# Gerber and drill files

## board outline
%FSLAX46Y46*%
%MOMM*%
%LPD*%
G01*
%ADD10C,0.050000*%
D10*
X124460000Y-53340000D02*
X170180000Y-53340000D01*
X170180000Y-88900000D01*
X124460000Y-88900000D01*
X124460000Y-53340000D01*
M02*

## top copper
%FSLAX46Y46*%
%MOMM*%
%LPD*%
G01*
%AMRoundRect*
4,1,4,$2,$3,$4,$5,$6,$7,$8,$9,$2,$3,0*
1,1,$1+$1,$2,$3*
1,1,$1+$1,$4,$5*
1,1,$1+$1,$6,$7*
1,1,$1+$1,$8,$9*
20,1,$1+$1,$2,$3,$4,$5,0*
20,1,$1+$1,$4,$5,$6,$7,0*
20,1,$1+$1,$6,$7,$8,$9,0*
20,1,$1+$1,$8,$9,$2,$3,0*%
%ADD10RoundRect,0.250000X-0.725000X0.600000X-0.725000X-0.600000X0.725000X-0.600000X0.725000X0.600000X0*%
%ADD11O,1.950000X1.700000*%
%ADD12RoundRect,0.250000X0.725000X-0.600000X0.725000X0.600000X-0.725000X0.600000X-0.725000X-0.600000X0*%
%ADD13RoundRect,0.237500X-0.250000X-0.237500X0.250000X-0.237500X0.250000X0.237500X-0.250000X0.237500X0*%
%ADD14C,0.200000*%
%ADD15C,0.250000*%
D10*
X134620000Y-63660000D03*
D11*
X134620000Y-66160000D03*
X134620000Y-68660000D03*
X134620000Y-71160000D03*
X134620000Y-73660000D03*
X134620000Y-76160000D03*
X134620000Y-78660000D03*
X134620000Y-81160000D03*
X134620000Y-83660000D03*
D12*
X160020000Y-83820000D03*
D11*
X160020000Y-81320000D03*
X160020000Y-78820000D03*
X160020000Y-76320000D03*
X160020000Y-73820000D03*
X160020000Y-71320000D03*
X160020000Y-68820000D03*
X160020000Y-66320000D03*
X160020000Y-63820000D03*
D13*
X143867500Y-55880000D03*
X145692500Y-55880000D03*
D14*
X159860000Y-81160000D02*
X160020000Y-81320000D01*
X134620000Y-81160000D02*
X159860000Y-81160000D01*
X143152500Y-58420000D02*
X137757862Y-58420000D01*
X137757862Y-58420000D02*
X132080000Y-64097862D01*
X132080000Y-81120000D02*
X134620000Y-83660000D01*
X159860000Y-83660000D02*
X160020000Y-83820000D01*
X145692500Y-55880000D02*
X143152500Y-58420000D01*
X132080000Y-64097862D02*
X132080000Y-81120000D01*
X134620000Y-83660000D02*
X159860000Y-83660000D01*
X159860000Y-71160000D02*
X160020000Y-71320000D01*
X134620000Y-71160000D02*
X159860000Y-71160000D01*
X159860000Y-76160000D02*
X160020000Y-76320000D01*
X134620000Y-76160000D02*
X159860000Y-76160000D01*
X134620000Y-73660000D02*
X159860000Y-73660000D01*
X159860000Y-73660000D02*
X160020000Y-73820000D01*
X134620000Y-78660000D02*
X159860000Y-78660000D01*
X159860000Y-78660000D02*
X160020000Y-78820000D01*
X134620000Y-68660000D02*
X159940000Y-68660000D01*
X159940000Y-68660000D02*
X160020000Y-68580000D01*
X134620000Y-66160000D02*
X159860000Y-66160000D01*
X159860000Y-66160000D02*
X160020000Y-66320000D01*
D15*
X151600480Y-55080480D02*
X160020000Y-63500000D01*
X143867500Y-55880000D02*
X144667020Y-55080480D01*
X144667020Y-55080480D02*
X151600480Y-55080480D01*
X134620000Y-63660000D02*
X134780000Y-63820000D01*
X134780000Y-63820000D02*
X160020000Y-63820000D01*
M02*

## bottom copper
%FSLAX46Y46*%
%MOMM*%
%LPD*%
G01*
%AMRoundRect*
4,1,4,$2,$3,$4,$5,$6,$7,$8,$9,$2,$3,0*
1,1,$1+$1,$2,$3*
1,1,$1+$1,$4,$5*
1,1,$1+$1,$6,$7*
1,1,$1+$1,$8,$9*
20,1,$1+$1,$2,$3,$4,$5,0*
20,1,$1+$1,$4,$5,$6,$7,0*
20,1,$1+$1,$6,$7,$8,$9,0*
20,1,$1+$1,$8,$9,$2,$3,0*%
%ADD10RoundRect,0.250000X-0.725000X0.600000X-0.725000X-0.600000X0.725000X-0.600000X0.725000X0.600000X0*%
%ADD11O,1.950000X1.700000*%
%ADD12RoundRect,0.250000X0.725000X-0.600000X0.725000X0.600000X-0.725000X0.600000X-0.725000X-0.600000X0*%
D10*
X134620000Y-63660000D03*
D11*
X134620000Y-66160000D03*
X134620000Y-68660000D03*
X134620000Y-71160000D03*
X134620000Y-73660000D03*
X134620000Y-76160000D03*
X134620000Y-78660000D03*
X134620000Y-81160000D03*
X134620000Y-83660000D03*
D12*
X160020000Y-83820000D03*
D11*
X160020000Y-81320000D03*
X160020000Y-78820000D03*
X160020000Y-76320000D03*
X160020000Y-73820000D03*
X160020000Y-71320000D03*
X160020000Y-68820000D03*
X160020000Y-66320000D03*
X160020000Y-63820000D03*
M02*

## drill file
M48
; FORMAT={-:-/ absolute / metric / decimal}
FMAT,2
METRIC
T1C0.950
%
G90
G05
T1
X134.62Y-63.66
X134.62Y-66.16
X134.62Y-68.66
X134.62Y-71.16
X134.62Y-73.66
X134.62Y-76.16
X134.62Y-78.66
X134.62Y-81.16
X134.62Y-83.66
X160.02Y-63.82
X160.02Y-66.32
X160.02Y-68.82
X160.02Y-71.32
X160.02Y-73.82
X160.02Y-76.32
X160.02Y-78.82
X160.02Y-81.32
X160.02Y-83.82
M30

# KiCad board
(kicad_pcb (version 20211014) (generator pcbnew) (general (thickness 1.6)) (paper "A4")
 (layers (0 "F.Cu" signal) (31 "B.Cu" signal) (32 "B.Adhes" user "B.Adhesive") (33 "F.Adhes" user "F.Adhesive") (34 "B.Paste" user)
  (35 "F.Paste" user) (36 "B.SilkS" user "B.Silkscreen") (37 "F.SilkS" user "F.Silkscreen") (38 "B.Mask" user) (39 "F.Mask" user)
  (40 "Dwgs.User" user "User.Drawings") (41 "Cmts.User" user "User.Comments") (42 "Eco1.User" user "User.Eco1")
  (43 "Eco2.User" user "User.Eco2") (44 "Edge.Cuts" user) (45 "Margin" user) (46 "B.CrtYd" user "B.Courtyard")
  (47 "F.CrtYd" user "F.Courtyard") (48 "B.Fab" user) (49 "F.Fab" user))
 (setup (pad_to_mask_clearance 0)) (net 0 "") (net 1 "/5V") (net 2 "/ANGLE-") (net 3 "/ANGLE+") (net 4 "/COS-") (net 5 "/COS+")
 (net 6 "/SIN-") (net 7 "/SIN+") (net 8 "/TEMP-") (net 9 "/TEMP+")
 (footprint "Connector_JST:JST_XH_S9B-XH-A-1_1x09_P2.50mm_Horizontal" (layer "F.Cu") (at 134.62 63.66 -90)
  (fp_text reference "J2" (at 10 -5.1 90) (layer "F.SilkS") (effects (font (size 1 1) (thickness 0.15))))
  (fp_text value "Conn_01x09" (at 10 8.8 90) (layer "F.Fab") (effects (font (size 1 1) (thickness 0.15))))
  (pad "1" thru_hole roundrect (at 0 0 270) (size 1.7 1.95) (drill 0.95) (layers *.Cu *.Mask) (roundrect_rratio 0.147059) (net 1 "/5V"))
  (pad "2" thru_hole oval (at 2.5 0 270) (size 1.7 1.95) (drill 0.95) (layers *.Cu *.Mask) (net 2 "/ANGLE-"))
  (pad "3" thru_hole oval (at 5 0 270) (size 1.7 1.95) (drill 0.95) (layers *.Cu *.Mask) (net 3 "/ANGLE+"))
  (pad "4" thru_hole oval (at 7.5 0 270) (size 1.7 1.95) (drill 0.95) (layers *.Cu *.Mask) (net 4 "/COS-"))
  (pad "5" thru_hole oval (at 10 0 270) (size 1.7 1.95) (drill 0.95) (layers *.Cu *.Mask) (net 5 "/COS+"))
  (pad "6" thru_hole oval (at 12.5 0 270) (size 1.7 1.95) (drill 0.95) (layers *.Cu *.Mask) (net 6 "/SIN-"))
  (pad "7" thru_hole oval (at 15 0 270) (size 1.7 1.95) (drill 0.95) (layers *.Cu *.Mask) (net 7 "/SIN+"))
  (pad "8" thru_hole oval (at 17.5 0 270) (size 1.7 1.95) (drill 0.95) (layers *.Cu *.Mask) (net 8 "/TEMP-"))
  (pad "9" thru_hole oval (at 20 0 270) (size 1.7 1.95) (drill 0.95) (layers *.Cu *.Mask) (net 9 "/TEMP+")))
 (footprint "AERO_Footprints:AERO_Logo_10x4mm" (layer "F.Cu") (at 147.32 60.96)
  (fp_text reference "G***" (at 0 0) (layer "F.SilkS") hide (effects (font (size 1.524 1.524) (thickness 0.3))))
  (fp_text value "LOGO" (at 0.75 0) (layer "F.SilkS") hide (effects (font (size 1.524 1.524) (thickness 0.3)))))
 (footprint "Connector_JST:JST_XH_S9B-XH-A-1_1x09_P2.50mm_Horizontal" (layer "F.Cu") (at 160.02 83.82 90)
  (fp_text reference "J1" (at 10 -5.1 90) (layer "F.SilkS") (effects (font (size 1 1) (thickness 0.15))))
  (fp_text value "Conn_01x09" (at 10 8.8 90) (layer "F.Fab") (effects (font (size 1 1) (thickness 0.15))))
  (pad "1" thru_hole roundrect (at 0 0 90) (size 1.7 1.95) (drill 0.95) (layers *.Cu *.Mask) (roundrect_rratio 0.147059) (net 9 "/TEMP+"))
  (pad "2" thru_hole oval (at 2.5 0 90) (size 1.7 1.95) (drill 0.95) (layers *.Cu *.Mask) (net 8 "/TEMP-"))
  (pad "3" thru_hole oval (at 5 0 90) (size 1.7 1.95) (drill 0.95) (layers *.Cu *.Mask) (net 7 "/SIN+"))
  (pad "4" thru_hole oval (at 7.5 0 90) (size 1.7 1.95) (drill 0.95) (layers *.Cu *.Mask) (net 6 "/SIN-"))
  (pad "5" thru_hole oval (at 10 0 90) (size 1.7 1.95) (drill 0.95) (layers *.Cu *.Mask) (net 5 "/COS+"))
  (pad "6" thru_hole oval (at 12.5 0 90) (size 1.7 1.95) (drill 0.95) (layers *.Cu *.Mask) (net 4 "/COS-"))
  (pad "7" thru_hole oval (at 15 0 90) (size 1.7 1.95) (drill 0.95) (layers *.Cu *.Mask) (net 3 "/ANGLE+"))
  (pad "8" thru_hole oval (at 17.5 0 90) (size 1.7 1.95) (drill 0.95) (layers *.Cu *.Mask) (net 2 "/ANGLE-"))
  (pad "9" thru_hole oval (at 20 0 90) (size 1.7 1.95) (drill 0.95) (layers *.Cu *.Mask) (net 1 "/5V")))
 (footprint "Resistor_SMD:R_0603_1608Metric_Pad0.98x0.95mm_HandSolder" (layer "F.Cu") (at 144.78 55.88)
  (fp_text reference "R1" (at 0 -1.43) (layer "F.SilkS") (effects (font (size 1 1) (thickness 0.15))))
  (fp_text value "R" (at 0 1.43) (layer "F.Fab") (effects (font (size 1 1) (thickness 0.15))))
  (pad "1" smd roundrect (at -0.9125 0) (size 0.975 0.95) (layers "F.Cu" "F.Paste" "F.Mask") (roundrect_rratio 0.25) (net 1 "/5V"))
  (pad "2" smd roundrect (at 0.9125 0) (size 0.975 0.95) (layers "F.Cu" "F.Paste" "F.Mask") (roundrect_rratio 0.25) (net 9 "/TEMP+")))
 (gr_rect (start 124.46 53.34) (end 170.18 88.9) (layer "Edge.Cuts") (width 0.05) (fill none))
 (segment (start 159.86 81.16) (end 160.02 81.32) (width 0.2) (layer "F.Cu") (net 8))
 (segment (start 134.62 81.16) (end 159.86 81.16) (width 0.2) (layer "F.Cu") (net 8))
 (segment (start 143.1525 58.42) (end 137.757862 58.42) (width 0.2) (layer "F.Cu") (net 9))
 (segment (start 137.757862 58.42) (end 132.08 64.097862) (width 0.2) (layer "F.Cu") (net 9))
 (segment (start 132.08 81.12) (end 134.62 83.66) (width 0.2) (layer "F.Cu") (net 9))
 (segment (start 159.86 83.66) (end 160.02 83.82) (width 0.2) (layer "F.Cu") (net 9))
 (segment (start 145.6925 55.88) (end 143.1525 58.42) (width 0.2) (layer "F.Cu") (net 9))
 (segment (start 132.08 64.097862) (end 132.08 81.12) (width 0.2) (layer "F.Cu") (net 9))
 (segment (start 134.62 83.66) (end 159.86 83.66) (width 0.2) (layer "F.Cu") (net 9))
 (segment (start 159.86 71.16) (end 160.02 71.32) (width 0.2) (layer "F.Cu") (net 4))
 (segment (start 134.62 71.16) (end 159.86 71.16) (width 0.2) (layer "F.Cu") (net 4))
 (segment (start 159.86 76.16) (end 160.02 76.32) (width 0.2) (layer "F.Cu") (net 6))
 (segment (start 134.62 76.16) (end 159.86 76.16) (width 0.2) (layer "F.Cu") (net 6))
 (segment (start 134.62 73.66) (end 159.86 73.66) (width 0.2) (layer "F.Cu") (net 5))
 (segment (start 159.86 73.66) (end 160.02 73.82) (width 0.2) (layer "F.Cu") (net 5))
 (segment (start 134.62 78.66) (end 159.86 78.66) (width 0.2) (layer "F.Cu") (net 7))
 (segment (start 159.86 78.66) (end 160.02 78.82) (width 0.2) (layer "F.Cu") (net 7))
 (segment (start 134.62 68.66) (end 159.94 68.66) (width 0.2) (layer "F.Cu") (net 3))
 (segment (start 159.94 68.66) (end 160.02 68.58) (width 0.2) (layer "F.Cu") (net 3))
 (segment (start 134.62 66.16) (end 159.86 66.16) (width 0.2) (layer "F.Cu") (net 2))
 (segment (start 159.86 66.16) (end 160.02 66.32) (width 0.2) (layer "F.Cu") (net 2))
 (segment (start 151.60048 55.08048) (end 160.02 63.5) (width 0.25) (layer "F.Cu") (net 1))
 (segment (start 143.8675 55.88) (end 144.66702 55.08048) (width 0.25) (layer "F.Cu") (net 1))
 (segment (start 144.66702 55.08048) (end 151.60048 55.08048) (width 0.25) (layer "F.Cu") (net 1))
 (segment (start 134.62 63.66) (end 134.78 63.82) (width 0.25) (layer "F.Cu") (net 1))
 (segment (start 134.78 63.82) (end 160.02 63.82) (width 0.25) (layer "F.Cu") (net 1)))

